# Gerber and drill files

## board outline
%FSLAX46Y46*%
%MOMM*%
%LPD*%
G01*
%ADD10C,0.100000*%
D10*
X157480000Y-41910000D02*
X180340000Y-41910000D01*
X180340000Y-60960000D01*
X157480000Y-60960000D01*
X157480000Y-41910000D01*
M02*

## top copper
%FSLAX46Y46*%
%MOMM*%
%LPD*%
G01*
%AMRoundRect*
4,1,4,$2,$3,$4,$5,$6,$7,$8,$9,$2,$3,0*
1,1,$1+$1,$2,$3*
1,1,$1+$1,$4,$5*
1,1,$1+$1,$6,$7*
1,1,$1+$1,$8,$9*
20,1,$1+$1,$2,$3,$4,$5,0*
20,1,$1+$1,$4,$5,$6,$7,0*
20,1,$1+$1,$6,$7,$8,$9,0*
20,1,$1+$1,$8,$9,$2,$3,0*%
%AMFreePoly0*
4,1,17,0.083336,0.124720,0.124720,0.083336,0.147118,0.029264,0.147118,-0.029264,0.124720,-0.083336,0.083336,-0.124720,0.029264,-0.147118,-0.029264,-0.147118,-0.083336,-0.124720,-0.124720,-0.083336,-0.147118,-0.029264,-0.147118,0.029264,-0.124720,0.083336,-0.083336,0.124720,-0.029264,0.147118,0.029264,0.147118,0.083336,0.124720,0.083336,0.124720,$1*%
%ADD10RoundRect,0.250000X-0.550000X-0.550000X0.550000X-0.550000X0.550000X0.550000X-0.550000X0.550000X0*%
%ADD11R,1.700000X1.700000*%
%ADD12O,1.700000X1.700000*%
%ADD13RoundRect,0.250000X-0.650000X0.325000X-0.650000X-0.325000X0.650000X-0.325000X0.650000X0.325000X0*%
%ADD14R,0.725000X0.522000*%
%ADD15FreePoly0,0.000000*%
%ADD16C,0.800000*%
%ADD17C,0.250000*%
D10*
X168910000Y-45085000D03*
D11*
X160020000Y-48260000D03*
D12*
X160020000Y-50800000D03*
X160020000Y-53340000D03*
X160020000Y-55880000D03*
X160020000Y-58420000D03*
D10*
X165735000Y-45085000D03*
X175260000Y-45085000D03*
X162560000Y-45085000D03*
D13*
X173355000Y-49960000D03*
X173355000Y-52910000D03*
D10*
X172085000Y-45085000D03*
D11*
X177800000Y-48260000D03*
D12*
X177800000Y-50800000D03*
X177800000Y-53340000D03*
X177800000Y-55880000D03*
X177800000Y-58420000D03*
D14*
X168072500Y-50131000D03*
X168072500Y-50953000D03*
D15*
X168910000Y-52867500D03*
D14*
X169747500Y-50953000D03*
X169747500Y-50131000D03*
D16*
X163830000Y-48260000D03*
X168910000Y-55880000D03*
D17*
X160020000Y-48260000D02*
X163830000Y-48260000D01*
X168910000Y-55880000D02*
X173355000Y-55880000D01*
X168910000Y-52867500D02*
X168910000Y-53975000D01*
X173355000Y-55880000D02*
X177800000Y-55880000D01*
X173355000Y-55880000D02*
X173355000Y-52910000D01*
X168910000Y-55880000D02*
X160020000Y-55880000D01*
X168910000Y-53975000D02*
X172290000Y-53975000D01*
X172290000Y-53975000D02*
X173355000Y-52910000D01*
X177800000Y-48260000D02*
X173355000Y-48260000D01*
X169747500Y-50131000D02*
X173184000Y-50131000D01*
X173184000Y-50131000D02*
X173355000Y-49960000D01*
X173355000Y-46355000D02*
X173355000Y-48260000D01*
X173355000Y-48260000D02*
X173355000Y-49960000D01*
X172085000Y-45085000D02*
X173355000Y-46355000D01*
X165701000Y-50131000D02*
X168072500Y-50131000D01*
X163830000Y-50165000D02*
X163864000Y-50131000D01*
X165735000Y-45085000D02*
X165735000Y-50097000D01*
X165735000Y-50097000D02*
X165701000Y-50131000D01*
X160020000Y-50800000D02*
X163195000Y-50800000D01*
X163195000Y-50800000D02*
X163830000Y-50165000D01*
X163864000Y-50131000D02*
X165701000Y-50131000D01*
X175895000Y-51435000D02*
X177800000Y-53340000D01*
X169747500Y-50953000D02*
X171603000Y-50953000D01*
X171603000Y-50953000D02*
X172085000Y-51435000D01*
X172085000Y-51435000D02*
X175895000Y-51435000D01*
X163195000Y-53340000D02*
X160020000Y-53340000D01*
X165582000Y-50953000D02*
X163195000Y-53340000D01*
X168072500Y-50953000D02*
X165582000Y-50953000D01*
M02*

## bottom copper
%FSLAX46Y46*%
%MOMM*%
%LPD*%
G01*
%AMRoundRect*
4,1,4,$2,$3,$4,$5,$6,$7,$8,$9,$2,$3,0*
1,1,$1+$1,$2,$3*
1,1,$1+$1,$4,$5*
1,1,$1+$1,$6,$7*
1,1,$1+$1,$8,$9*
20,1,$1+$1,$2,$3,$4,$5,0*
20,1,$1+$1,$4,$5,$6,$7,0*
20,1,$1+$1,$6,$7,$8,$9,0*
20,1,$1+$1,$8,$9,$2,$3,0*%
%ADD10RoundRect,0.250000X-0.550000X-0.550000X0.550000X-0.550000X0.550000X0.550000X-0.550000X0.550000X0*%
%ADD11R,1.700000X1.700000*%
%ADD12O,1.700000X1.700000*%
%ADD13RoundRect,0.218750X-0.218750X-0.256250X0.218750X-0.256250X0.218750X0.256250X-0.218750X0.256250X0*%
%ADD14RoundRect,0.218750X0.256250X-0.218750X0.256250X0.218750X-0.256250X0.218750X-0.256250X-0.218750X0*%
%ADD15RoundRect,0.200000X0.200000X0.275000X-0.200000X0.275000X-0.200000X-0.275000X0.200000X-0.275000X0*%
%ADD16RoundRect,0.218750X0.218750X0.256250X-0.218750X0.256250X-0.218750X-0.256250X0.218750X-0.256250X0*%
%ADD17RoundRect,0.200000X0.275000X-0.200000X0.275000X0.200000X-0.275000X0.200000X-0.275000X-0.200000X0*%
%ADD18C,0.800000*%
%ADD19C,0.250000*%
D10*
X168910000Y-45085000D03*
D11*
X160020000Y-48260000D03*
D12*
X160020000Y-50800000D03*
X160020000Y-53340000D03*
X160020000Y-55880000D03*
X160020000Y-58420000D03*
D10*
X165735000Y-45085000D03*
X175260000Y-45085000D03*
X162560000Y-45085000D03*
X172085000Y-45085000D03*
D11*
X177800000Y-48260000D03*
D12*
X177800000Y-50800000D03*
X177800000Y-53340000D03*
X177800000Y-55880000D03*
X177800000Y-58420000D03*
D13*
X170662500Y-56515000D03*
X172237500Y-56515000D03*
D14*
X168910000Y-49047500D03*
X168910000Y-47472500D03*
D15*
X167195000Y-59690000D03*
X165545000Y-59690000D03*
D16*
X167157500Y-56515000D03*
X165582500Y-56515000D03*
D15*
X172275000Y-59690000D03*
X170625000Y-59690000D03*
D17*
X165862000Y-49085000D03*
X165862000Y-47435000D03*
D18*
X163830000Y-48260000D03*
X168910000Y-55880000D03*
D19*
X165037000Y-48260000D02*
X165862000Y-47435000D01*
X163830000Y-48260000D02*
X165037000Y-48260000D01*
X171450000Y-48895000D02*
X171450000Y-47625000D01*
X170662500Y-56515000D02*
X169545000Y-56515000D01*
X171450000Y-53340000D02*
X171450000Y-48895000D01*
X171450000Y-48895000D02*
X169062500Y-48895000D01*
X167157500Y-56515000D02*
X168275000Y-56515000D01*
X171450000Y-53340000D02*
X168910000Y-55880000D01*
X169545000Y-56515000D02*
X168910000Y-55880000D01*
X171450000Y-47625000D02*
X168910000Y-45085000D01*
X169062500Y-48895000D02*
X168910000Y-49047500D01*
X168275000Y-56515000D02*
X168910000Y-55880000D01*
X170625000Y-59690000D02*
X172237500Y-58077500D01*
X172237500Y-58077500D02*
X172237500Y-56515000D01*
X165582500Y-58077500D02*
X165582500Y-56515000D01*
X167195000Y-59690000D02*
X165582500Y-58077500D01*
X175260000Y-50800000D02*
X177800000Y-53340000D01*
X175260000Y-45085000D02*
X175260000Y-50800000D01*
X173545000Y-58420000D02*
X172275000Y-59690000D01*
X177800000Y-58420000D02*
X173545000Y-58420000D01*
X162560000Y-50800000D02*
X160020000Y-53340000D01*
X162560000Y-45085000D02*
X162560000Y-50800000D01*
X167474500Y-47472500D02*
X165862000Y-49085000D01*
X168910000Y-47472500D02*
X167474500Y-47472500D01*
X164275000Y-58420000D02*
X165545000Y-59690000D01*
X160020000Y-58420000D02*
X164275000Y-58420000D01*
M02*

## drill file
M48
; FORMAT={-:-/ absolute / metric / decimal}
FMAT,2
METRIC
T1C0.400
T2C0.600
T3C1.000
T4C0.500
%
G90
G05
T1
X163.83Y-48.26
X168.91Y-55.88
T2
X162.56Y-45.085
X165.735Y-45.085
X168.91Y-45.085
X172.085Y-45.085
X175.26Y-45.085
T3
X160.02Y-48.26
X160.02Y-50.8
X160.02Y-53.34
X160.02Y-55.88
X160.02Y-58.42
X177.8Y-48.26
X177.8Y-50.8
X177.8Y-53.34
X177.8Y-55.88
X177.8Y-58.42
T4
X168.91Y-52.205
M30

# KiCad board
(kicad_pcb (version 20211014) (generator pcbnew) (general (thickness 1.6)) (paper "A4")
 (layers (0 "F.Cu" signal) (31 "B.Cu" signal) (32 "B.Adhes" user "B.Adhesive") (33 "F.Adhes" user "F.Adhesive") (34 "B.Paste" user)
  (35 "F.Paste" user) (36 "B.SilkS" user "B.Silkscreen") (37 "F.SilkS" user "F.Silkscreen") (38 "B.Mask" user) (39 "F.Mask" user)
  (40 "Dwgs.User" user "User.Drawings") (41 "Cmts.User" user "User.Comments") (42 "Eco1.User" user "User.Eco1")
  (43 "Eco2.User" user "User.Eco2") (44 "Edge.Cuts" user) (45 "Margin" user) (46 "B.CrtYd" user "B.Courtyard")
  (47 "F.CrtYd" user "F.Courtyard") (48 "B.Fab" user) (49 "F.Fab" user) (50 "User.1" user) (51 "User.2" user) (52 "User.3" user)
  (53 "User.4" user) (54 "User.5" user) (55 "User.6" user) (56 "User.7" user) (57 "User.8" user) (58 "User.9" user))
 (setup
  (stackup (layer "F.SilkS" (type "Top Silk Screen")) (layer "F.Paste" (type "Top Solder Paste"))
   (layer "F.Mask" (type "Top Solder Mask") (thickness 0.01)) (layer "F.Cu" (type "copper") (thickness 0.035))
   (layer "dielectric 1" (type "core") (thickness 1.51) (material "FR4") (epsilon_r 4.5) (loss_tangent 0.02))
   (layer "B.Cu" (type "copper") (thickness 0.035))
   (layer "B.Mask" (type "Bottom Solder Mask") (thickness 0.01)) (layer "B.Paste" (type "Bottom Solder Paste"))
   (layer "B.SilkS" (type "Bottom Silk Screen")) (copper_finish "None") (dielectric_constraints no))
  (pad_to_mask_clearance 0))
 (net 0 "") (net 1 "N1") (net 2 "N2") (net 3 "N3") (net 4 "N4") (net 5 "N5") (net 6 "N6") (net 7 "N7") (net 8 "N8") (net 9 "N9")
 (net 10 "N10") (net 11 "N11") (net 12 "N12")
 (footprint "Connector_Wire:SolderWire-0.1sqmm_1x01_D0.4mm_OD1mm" (layer "F.Cu") (at 168.91 45.085)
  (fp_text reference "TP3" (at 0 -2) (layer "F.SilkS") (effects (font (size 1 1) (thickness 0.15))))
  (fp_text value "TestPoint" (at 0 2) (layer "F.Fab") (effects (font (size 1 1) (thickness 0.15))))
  (pad "1" thru_hole roundrect (at 0 0) (size 1.6 1.6) (drill 0.6) (layers *.Cu *.Mask) (roundrect_rratio 0.15625) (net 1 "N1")))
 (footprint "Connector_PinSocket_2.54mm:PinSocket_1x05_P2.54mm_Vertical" (layer "F.Cu") (at 160.02 48.26)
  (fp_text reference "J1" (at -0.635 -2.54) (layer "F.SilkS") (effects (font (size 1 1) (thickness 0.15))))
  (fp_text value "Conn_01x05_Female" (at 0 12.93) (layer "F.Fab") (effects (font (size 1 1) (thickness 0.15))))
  (pad "1" thru_hole rect (at 0 0) (size 1.7 1.7) (drill 1) (layers *.Cu *.Mask) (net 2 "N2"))
  (pad "2" thru_hole oval (at 0 2.54) (size 1.7 1.7) (drill 1) (layers *.Cu *.Mask) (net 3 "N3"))
  (pad "3" thru_hole oval (at 0 5.08) (size 1.7 1.7) (drill 1) (layers *.Cu *.Mask) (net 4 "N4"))
  (pad "4" thru_hole oval (at 0 7.62) (size 1.7 1.7) (drill 1) (layers *.Cu *.Mask) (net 1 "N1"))
  (pad "5" thru_hole oval (at 0 10.16) (size 1.7 1.7) (drill 1) (layers *.Cu *.Mask) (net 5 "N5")))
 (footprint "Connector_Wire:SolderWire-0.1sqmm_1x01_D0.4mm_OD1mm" (layer "F.Cu") (at 165.735 45.085)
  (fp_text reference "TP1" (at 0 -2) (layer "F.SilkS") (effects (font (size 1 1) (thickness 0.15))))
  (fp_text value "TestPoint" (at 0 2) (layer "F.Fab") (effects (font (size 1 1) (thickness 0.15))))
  (pad "1" thru_hole roundrect (at 0 0) (size 1.6 1.6) (drill 0.6) (layers *.Cu *.Mask) (roundrect_rratio 0.15625) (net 3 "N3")))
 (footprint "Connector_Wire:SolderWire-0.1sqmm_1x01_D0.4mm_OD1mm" (layer "F.Cu") (at 175.26 45.085)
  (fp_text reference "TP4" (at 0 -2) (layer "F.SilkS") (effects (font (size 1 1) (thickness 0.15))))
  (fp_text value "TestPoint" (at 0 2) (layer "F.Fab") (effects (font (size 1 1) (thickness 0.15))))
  (pad "1" thru_hole roundrect (at 0 0) (size 1.6 1.6) (drill 0.6) (layers *.Cu *.Mask) (roundrect_rratio 0.15625) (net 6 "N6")))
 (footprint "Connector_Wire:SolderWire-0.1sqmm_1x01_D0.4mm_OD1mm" (layer "F.Cu") (at 162.56 45.085)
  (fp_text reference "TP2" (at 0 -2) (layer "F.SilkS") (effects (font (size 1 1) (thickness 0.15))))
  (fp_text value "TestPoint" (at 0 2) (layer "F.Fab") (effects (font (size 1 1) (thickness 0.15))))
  (pad "1" thru_hole roundrect (at 0 0) (size 1.6 1.6) (drill 0.6) (layers *.Cu *.Mask) (roundrect_rratio 0.15625) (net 4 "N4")))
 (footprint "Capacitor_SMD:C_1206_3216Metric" (layer "F.Cu") (at 173.355 51.435 -90)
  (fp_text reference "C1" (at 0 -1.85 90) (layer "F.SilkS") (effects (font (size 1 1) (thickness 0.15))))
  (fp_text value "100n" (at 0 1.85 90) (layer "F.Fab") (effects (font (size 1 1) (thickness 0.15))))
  (pad "1" smd roundrect (at -1.475 0 270) (size 1.15 1.8) (layers "F.Cu" "F.Paste" "F.Mask") (roundrect_rratio 0.2173913043) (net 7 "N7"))
  (pad "2" smd roundrect (at 1.475 0 270) (size 1.15 1.8) (layers "F.Cu" "F.Paste" "F.Mask") (roundrect_rratio 0.2173913043) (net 1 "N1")))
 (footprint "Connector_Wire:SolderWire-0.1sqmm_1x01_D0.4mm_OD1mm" (layer "F.Cu") (at 172.085 45.085)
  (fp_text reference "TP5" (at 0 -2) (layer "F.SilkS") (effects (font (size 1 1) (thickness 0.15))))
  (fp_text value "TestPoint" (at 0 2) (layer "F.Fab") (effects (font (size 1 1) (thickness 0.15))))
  (pad "1" thru_hole roundrect (at 0 0) (size 1.6 1.6) (drill 0.6) (layers *.Cu *.Mask) (roundrect_rratio 0.15625) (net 7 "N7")))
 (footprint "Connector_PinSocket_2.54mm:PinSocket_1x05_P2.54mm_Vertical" (layer "F.Cu") (at 177.8 48.26)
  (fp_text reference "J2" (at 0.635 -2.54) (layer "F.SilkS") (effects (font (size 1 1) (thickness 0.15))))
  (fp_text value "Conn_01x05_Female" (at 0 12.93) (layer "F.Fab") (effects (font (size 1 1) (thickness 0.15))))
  (pad "1" thru_hole rect (at 0 0) (size 1.7 1.7) (drill 1) (layers *.Cu *.Mask) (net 7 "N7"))
  (pad "2" thru_hole oval (at 0 2.54) (size 1.7 1.7) (drill 1) (layers *.Cu *.Mask) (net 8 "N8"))
  (pad "3" thru_hole oval (at 0 5.08) (size 1.7 1.7) (drill 1) (layers *.Cu *.Mask) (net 6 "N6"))
  (pad "4" thru_hole oval (at 0 7.62) (size 1.7 1.7) (drill 1) (layers *.Cu *.Mask) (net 1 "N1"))
  (pad "5" thru_hole oval (at 0 10.16) (size 1.7 1.7) (drill 1) (layers *.Cu *.Mask) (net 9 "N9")))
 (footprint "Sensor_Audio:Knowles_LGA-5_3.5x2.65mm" (layer "F.Cu") (at 168.91 51.435)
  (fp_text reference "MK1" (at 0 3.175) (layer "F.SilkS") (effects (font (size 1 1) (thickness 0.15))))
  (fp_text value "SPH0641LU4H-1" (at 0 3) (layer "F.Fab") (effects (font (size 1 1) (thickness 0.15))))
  (pad "" np_thru_hole circle (at 0 0.77) (size 0.5 0.5) (drill 0.5) (layers *.Cu *.Mask))
  (pad "1" smd rect (at -0.8375 -1.304) (size 0.725 0.522) (layers "F.Cu" "F.Paste" "F.Mask") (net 3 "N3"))
  (pad "2" smd rect (at -0.8375 -0.482) (size 0.725 0.522) (layers "F.Cu" "F.Paste" "F.Mask") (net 4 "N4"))
  (pad "3" smd custom (at 0 1.4325) (size 0.3 0.3) (layers "F.Cu" "F.Mask") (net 1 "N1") (zone_connect 0)
   (options (clearance outline) (anchor circle)) (primitives))
  (pad "4" smd rect (at 0.8375 -0.482) (size 0.725 0.522) (layers "F.Cu" "F.Paste" "F.Mask") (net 6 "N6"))
  (pad "5" smd rect (at 0.8375 -1.304) (size 0.725 0.522) (layers "F.Cu" "F.Paste" "F.Mask") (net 7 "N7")))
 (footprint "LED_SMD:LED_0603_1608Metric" (layer "B.Cu") (at 171.45 56.515)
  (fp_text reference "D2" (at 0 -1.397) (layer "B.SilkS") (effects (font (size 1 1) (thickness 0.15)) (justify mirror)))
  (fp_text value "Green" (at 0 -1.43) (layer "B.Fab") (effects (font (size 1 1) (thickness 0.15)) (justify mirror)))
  (pad "1" smd roundrect (at -0.7875 0) (size 0.875 0.95) (layers "B.Cu" "B.Paste" "B.Mask") (roundrect_rratio 0.25) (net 1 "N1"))
  (pad "2" smd roundrect (at 0.7875 0) (size 0.875 0.95) (layers "B.Cu" "B.Paste" "B.Mask") (roundrect_rratio 0.25) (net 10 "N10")))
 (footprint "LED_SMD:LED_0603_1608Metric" (layer "B.Cu") (at 168.91 48.26 90)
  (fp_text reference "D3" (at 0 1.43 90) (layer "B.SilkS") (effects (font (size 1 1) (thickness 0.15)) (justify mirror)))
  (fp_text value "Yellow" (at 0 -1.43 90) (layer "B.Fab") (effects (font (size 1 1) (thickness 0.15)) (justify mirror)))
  (pad "1" smd roundrect (at -0.7875 0 90) (size 0.875 0.95) (layers "B.Cu" "B.Paste" "B.Mask") (roundrect_rratio 0.25) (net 1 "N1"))
  (pad "2" smd roundrect (at 0.7875 0 90) (size 0.875 0.95) (layers "B.Cu" "B.Paste" "B.Mask") (roundrect_rratio 0.25) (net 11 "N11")))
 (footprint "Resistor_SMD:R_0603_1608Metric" (layer "B.Cu") (at 166.37 59.69 180)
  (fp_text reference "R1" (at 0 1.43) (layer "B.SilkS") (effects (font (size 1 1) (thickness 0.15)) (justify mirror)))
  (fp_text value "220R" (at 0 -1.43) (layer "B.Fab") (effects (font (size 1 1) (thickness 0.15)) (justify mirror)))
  (pad "1" smd roundrect (at -0.825 0 180) (size 0.8 0.95) (layers "B.Cu" "B.Paste" "B.Mask") (roundrect_rratio 0.25) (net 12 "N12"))
  (pad "2" smd roundrect (at 0.825 0 180) (size 0.8 0.95) (layers "B.Cu" "B.Paste" "B.Mask") (roundrect_rratio 0.25) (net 5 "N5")))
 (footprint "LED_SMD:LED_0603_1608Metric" (layer "B.Cu") (at 166.37 56.515 180)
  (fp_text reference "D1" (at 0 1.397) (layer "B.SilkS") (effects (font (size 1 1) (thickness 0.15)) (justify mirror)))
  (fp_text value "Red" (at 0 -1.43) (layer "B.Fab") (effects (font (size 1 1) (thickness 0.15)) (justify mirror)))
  (pad "1" smd roundrect (at -0.7875 0 180) (size 0.875 0.95) (layers "B.Cu" "B.Paste" "B.Mask") (roundrect_rratio 0.25) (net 1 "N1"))
  (pad "2" smd roundrect (at 0.7875 0 180) (size 0.875 0.95) (layers "B.Cu" "B.Paste" "B.Mask") (roundrect_rratio 0.25) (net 12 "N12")))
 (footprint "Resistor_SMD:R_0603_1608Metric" (layer "B.Cu") (at 171.45 59.69 180)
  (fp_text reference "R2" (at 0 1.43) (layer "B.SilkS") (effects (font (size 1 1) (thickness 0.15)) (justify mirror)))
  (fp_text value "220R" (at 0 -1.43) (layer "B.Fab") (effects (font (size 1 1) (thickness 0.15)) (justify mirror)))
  (pad "1" smd roundrect (at -0.825 0 180) (size 0.8 0.95) (layers "B.Cu" "B.Paste" "B.Mask") (roundrect_rratio 0.25) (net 9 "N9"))
  (pad "2" smd roundrect (at 0.825 0 180) (size 0.8 0.95) (layers "B.Cu" "B.Paste" "B.Mask") (roundrect_rratio 0.25) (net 10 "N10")))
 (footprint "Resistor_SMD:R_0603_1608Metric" (layer "B.Cu") (at 165.862 48.26 90)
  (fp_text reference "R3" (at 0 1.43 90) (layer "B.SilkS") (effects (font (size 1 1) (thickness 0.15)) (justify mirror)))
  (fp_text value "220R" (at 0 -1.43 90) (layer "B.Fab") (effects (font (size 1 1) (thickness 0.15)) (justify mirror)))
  (pad "1" smd roundrect (at -0.825 0 90) (size 0.8 0.95) (layers "B.Cu" "B.Paste" "B.Mask") (roundrect_rratio 0.25) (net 11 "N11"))
  (pad "2" smd roundrect (at 0.825 0 90) (size 0.8 0.95) (layers "B.Cu" "B.Paste" "B.Mask") (roundrect_rratio 0.25) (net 2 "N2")))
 (gr_rect (start 180.34 60.96) (end 157.48 41.91) (layer "Edge.Cuts") (width 0.1) (fill none))
 (segment (start 160.02 48.26) (end 163.83 48.26) (width 0.25) (layer "F.Cu") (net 2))
 (via (at 163.83 48.26) (size 0.8) (drill 0.4) (layers "F.Cu" "B.Cu") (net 2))
 (segment (start 165.037 48.26) (end 165.862 47.435) (width 0.25) (layer "B.Cu") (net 2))
 (segment (start 163.83 48.26) (end 165.037 48.26) (width 0.25) (layer "B.Cu") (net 2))
 (segment (start 168.91 55.88) (end 173.355 55.88) (width 0.25) (layer "F.Cu") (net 1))
 (segment (start 168.91 52.8675) (end 168.91 53.975) (width 0.25) (layer "F.Cu") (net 1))
 (segment (start 173.355 55.88) (end 177.8 55.88) (width 0.25) (layer "F.Cu") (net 1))
 (segment (start 173.355 55.88) (end 173.355 52.91) (width 0.25) (layer "F.Cu") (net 1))
 (segment (start 168.91 55.88) (end 160.02 55.88) (width 0.25) (layer "F.Cu") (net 1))
 (segment (start 168.91 53.975) (end 172.29 53.975) (width 0.25) (layer "F.Cu") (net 1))
 (segment (start 172.29 53.975) (end 173.355 52.91) (width 0.25) (layer "F.Cu") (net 1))
 (via (at 168.91 55.88) (size 0.8) (drill 0.4) (layers "F.Cu" "B.Cu") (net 1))
 (segment (start 171.45 48.895) (end 171.45 47.625) (width 0.25) (layer "B.Cu") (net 1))
 (segment (start 170.6625 56.515) (end 169.545 56.515) (width 0.25) (layer "B.Cu") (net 1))
 (segment (start 171.45 53.34) (end 171.45 48.895) (width 0.25) (layer "B.Cu") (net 1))
 (segment (start 171.45 48.895) (end 169.0625 48.895) (width 0.25) (layer "B.Cu") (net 1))
 (segment (start 167.1575 56.515) (end 168.275 56.515) (width 0.25) (layer "B.Cu") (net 1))
 (segment (start 171.45 53.34) (end 168.91 55.88) (width 0.25) (layer "B.Cu") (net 1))
 (segment (start 169.545 56.515) (end 168.91 55.88) (width 0.25) (layer "B.Cu") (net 1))
 (segment (start 171.45 47.625) (end 168.91 45.085) (width 0.25) (layer "B.Cu") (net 1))
 (segment (start 169.0625 48.895) (end 168.91 49.0475) (width 0.25) (layer "B.Cu") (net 1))
 (segment (start 168.275 56.515) (end 168.91 55.88) (width 0.25) (layer "B.Cu") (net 1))
 (segment (start 177.8 48.26) (end 173.355 48.26) (width 0.25) (layer "F.Cu") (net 7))
 (segment (start 169.7475 50.131) (end 173.184 50.131) (width 0.25) (layer "F.Cu") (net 7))
 (segment (start 173.184 50.131) (end 173.355 49.96) (width 0.25) (layer "F.Cu") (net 7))
 (segment (start 173.355 46.355) (end 173.355 48.26) (width 0.25) (layer "F.Cu") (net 7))
 (segment (start 173.355 48.26) (end 173.355 49.96) (width 0.25) (layer "F.Cu") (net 7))
 (segment (start 172.085 45.085) (end 173.355 46.355) (width 0.25) (layer "F.Cu") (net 7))
 (segment (start 170.625 59.69) (end 172.2375 58.0775) (width 0.25) (layer "B.Cu") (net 10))
 (segment (start 172.2375 58.0775) (end 172.2375 56.515) (width 0.25) (layer "B.Cu") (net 10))
 (segment (start 165.701 50.131) (end 168.0725 50.131) (width 0.25) (layer "F.Cu") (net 3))
 (segment (start 163.83 50.165) (end 163.864 50.131) (width 0.25) (layer "F.Cu") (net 3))
 (segment (start 165.735 45.085) (end 165.735 50.097) (width 0.25) (layer "F.Cu") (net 3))
 (segment (start 165.735 50.097) (end 165.701 50.131) (width 0.25) (layer "F.Cu") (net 3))
 (segment (start 160.02 50.8) (end 163.195 50.8) (width 0.25) (layer "F.Cu") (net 3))
 (segment (start 163.195 50.8) (end 163.83 50.165) (width 0.25) (layer "F.Cu") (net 3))
 (segment (start 163.864 50.131) (end 165.701 50.131) (width 0.25) (layer "F.Cu") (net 3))
 (segment (start 165.5825 58.0775) (end 165.5825 56.515) (width 0.25) (layer "B.Cu") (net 12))
 (segment (start 167.195 59.69) (end 165.5825 58.0775) (width 0.25) (layer "B.Cu") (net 12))
 (segment (start 175.895 51.435) (end 177.8 53.34) (width 0.25) (layer "F.Cu") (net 6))
 (segment (start 169.7475 50.953) (end 171.603 50.953) (width 0.25) (layer "F.Cu") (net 6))
 (segment (start 171.603 50.953) (end 172.085 51.435) (width 0.25) (layer "F.Cu") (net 6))
 (segment (start 172.085 51.435) (end 175.895 51.435) (width 0.25) (layer "F.Cu") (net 6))
 (segment (start 175.26 50.8) (end 177.8 53.34) (width 0.25) (layer "B.Cu") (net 6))
 (segment (start 175.26 45.085) (end 175.26 50.8) (width 0.25) (layer "B.Cu") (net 6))
 (segment (start 173.545 58.42) (end 172.275 59.69) (width 0.25) (layer "B.Cu") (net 9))
 (segment (start 177.8 58.42) (end 173.545 58.42) (width 0.25) (layer "B.Cu") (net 9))
 (segment (start 163.195 53.34) (end 160.02 53.34) (width 0.25) (layer "F.Cu") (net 4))
 (segment (start 165.582 50.953) (end 163.195 53.34) (width 0.25) (layer "F.Cu") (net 4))
 (segment (start 168.0725 50.953) (end 165.582 50.953) (width 0.25) (layer "F.Cu") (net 4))
 (segment (start 162.56 50.8) (end 160.02 53.34) (width 0.25) (layer "B.Cu") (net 4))
 (segment (start 162.56 45.085) (end 162.56 50.8) (width 0.25) (layer "B.Cu") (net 4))
 (segment (start 167.4745 47.4725) (end 165.862 49.085) (width 0.25) (layer "B.Cu") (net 11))
 (segment (start 168.91 47.4725) (end 167.4745 47.4725) (width 0.25) (layer "B.Cu") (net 11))
 (segment (start 164.275 58.42) (end 165.545 59.69) (width 0.25) (layer "B.Cu") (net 5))
 (segment (start 160.02 58.42) (end 164.275 58.42) (width 0.25) (layer "B.Cu") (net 5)))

